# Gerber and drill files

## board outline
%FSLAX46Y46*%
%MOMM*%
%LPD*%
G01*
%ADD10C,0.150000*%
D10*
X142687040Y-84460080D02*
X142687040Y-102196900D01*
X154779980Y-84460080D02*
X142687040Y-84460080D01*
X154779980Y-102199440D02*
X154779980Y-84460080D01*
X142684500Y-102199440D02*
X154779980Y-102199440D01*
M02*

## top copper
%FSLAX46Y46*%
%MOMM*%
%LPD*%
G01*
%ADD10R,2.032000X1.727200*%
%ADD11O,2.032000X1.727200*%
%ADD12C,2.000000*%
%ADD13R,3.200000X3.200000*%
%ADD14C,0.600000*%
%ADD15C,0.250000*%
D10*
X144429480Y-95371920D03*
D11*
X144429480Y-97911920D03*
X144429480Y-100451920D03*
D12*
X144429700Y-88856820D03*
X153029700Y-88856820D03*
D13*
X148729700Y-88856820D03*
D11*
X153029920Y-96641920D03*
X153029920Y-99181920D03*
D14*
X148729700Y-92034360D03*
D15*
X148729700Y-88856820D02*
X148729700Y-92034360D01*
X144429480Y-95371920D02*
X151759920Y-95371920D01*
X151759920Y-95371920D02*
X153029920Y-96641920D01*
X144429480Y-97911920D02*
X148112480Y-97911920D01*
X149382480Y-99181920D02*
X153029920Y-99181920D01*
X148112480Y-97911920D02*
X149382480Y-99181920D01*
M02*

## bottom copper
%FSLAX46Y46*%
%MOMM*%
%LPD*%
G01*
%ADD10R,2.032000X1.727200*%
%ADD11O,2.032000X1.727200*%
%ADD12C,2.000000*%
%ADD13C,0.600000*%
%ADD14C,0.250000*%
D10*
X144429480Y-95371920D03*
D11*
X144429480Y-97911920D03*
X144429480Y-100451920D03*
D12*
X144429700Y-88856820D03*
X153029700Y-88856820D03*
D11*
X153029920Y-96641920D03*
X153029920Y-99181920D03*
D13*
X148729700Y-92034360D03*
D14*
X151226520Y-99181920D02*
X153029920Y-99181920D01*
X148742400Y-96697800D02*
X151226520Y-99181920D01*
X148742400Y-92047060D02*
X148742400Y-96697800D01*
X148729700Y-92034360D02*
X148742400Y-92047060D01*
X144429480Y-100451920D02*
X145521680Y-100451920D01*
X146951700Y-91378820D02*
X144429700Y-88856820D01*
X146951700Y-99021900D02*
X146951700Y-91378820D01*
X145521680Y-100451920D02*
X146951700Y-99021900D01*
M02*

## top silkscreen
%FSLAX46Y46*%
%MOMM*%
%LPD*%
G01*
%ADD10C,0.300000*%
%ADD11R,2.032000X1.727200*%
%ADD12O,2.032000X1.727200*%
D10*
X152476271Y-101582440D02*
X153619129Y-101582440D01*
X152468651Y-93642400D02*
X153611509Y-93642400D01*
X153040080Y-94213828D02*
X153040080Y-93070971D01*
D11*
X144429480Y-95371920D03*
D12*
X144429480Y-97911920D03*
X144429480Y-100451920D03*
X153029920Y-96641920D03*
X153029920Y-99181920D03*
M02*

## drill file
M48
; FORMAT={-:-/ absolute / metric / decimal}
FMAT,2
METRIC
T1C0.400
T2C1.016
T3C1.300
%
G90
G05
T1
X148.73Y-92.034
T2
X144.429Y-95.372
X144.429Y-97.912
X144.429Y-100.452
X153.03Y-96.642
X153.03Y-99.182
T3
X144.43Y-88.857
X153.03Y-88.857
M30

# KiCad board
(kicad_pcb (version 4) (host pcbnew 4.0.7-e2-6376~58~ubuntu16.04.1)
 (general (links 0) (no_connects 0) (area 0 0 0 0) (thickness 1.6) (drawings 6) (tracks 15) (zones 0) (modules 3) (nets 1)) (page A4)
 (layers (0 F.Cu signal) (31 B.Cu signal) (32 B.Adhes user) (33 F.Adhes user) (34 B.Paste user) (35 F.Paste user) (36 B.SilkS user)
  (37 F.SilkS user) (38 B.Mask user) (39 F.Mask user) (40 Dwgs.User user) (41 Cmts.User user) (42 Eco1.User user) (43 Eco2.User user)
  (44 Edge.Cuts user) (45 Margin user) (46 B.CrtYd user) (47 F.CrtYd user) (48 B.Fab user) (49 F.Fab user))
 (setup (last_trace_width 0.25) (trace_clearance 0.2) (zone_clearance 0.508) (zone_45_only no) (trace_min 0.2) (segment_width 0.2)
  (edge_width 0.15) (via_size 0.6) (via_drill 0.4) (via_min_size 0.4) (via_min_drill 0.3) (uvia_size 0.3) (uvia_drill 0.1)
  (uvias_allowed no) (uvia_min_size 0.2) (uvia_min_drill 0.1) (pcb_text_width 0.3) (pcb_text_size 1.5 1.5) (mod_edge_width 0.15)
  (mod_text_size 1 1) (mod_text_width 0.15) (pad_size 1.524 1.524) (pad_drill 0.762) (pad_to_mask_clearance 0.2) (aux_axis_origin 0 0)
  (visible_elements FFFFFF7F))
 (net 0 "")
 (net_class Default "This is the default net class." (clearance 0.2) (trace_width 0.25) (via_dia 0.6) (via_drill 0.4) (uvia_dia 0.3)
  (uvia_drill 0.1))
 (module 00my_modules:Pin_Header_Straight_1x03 (layer F.Cu) (at 144.42948 95.37192)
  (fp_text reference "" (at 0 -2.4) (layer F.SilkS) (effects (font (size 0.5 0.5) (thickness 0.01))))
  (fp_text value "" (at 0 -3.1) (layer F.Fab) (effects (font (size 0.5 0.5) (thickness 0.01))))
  (pad 1 thru_hole rect (at 0 0) (size 2.032 1.7272) (drill 1.016) (layers *.Cu *.Mask F.SilkS))
  (pad 2 thru_hole oval (at 0 2.54) (size 2.032 1.7272) (drill 1.016) (layers *.Cu *.Mask F.SilkS))
  (pad 3 thru_hole oval (at 0 5.08) (size 2.032 1.7272) (drill 1.016) (layers *.Cu *.Mask F.SilkS)))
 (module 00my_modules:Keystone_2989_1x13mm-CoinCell (layer F.Cu) (at 148.7297 88.85682)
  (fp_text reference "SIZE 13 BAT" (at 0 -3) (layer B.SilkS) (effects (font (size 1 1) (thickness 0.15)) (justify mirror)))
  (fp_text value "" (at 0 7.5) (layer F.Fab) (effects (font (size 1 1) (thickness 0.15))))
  (pad 1 thru_hole circle (at -4.3 0) (size 2 2) (drill 1.3) (layers *.Cu *.Mask))
  (pad 1 thru_hole circle (at 4.3 0) (size 2 2) (drill 1.3) (layers *.Cu *.Mask))
  (pad 2 smd rect (at 0 0) (size 3.2 3.2) (layers F.Cu F.Mask)))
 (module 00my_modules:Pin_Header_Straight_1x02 (layer F.Cu) (at 153.02992 96.64192)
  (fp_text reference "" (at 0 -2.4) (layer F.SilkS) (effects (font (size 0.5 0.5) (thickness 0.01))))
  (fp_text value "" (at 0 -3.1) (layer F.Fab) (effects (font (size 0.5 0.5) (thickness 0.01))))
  (pad 1 thru_hole oval (at 0 0) (size 2.032 1.7272) (drill 1.016) (layers *.Cu *.Mask F.SilkS))
  (pad 2 thru_hole oval (at 0 2.54) (size 2.032 1.7272) (drill 1.016) (layers *.Cu *.Mask F.SilkS)))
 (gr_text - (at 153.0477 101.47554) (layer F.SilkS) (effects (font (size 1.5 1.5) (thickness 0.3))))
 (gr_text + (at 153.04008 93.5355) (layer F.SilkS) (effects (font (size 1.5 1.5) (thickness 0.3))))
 (gr_line (start 142.68704 84.46008) (end 142.68704 102.1969) (angle 90) (layer Edge.Cuts) (width 0.15))
 (gr_line (start 154.77998 84.46008) (end 142.68704 84.46008) (angle 90) (layer Edge.Cuts) (width 0.15))
 (gr_line (start 154.77998 102.19944) (end 154.77998 84.46008) (angle 90) (layer Edge.Cuts) (width 0.15))
 (gr_line (start 142.6845 102.19944) (end 154.77998 102.19944) (angle 90) (layer Edge.Cuts) (width 0.15))
 (segment (start 148.7297 88.85682) (end 148.7297 92.03436) (width 0.25) (layer F.Cu) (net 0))
 (segment (start 151.22652 99.18192) (end 153.02992 99.18192) (width 0.25) (layer B.Cu) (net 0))
 (segment (start 148.7424 96.6978) (end 151.22652 99.18192) (width 0.25) (layer B.Cu) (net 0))
 (segment (start 148.7424 92.04706) (end 148.7424 96.6978) (width 0.25) (layer B.Cu) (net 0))
 (segment (start 148.7297 92.03436) (end 148.7424 92.04706) (width 0.25) (layer B.Cu) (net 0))
 (via (at 148.7297 92.03436) (size 0.6) (drill 0.4) (layers F.Cu B.Cu) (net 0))
 (segment (start 144.42948 100.45192) (end 145.52168 100.45192) (width 0.25) (layer B.Cu) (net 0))
 (segment (start 146.9517 91.37882) (end 144.4297 88.85682) (width 0.25) (layer B.Cu) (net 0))
 (segment (start 146.9517 99.0219) (end 146.9517 91.37882) (width 0.25) (layer B.Cu) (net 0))
 (segment (start 145.52168 100.45192) (end 146.9517 99.0219) (width 0.25) (layer B.Cu) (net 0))
 (segment (start 144.42948 95.37192) (end 151.75992 95.37192) (width 0.25) (layer F.Cu) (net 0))
 (segment (start 151.75992 95.37192) (end 153.02992 96.64192) (width 0.25) (layer F.Cu) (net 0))
 (segment (start 144.42948 97.91192) (end 148.11248 97.91192) (width 0.25) (layer F.Cu) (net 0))
 (segment (start 149.38248 99.18192) (end 153.02992 99.18192) (width 0.25) (layer F.Cu) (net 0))
 (segment (start 148.11248 97.91192) (end 149.38248 99.18192) (width 0.25) (layer F.Cu) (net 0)))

